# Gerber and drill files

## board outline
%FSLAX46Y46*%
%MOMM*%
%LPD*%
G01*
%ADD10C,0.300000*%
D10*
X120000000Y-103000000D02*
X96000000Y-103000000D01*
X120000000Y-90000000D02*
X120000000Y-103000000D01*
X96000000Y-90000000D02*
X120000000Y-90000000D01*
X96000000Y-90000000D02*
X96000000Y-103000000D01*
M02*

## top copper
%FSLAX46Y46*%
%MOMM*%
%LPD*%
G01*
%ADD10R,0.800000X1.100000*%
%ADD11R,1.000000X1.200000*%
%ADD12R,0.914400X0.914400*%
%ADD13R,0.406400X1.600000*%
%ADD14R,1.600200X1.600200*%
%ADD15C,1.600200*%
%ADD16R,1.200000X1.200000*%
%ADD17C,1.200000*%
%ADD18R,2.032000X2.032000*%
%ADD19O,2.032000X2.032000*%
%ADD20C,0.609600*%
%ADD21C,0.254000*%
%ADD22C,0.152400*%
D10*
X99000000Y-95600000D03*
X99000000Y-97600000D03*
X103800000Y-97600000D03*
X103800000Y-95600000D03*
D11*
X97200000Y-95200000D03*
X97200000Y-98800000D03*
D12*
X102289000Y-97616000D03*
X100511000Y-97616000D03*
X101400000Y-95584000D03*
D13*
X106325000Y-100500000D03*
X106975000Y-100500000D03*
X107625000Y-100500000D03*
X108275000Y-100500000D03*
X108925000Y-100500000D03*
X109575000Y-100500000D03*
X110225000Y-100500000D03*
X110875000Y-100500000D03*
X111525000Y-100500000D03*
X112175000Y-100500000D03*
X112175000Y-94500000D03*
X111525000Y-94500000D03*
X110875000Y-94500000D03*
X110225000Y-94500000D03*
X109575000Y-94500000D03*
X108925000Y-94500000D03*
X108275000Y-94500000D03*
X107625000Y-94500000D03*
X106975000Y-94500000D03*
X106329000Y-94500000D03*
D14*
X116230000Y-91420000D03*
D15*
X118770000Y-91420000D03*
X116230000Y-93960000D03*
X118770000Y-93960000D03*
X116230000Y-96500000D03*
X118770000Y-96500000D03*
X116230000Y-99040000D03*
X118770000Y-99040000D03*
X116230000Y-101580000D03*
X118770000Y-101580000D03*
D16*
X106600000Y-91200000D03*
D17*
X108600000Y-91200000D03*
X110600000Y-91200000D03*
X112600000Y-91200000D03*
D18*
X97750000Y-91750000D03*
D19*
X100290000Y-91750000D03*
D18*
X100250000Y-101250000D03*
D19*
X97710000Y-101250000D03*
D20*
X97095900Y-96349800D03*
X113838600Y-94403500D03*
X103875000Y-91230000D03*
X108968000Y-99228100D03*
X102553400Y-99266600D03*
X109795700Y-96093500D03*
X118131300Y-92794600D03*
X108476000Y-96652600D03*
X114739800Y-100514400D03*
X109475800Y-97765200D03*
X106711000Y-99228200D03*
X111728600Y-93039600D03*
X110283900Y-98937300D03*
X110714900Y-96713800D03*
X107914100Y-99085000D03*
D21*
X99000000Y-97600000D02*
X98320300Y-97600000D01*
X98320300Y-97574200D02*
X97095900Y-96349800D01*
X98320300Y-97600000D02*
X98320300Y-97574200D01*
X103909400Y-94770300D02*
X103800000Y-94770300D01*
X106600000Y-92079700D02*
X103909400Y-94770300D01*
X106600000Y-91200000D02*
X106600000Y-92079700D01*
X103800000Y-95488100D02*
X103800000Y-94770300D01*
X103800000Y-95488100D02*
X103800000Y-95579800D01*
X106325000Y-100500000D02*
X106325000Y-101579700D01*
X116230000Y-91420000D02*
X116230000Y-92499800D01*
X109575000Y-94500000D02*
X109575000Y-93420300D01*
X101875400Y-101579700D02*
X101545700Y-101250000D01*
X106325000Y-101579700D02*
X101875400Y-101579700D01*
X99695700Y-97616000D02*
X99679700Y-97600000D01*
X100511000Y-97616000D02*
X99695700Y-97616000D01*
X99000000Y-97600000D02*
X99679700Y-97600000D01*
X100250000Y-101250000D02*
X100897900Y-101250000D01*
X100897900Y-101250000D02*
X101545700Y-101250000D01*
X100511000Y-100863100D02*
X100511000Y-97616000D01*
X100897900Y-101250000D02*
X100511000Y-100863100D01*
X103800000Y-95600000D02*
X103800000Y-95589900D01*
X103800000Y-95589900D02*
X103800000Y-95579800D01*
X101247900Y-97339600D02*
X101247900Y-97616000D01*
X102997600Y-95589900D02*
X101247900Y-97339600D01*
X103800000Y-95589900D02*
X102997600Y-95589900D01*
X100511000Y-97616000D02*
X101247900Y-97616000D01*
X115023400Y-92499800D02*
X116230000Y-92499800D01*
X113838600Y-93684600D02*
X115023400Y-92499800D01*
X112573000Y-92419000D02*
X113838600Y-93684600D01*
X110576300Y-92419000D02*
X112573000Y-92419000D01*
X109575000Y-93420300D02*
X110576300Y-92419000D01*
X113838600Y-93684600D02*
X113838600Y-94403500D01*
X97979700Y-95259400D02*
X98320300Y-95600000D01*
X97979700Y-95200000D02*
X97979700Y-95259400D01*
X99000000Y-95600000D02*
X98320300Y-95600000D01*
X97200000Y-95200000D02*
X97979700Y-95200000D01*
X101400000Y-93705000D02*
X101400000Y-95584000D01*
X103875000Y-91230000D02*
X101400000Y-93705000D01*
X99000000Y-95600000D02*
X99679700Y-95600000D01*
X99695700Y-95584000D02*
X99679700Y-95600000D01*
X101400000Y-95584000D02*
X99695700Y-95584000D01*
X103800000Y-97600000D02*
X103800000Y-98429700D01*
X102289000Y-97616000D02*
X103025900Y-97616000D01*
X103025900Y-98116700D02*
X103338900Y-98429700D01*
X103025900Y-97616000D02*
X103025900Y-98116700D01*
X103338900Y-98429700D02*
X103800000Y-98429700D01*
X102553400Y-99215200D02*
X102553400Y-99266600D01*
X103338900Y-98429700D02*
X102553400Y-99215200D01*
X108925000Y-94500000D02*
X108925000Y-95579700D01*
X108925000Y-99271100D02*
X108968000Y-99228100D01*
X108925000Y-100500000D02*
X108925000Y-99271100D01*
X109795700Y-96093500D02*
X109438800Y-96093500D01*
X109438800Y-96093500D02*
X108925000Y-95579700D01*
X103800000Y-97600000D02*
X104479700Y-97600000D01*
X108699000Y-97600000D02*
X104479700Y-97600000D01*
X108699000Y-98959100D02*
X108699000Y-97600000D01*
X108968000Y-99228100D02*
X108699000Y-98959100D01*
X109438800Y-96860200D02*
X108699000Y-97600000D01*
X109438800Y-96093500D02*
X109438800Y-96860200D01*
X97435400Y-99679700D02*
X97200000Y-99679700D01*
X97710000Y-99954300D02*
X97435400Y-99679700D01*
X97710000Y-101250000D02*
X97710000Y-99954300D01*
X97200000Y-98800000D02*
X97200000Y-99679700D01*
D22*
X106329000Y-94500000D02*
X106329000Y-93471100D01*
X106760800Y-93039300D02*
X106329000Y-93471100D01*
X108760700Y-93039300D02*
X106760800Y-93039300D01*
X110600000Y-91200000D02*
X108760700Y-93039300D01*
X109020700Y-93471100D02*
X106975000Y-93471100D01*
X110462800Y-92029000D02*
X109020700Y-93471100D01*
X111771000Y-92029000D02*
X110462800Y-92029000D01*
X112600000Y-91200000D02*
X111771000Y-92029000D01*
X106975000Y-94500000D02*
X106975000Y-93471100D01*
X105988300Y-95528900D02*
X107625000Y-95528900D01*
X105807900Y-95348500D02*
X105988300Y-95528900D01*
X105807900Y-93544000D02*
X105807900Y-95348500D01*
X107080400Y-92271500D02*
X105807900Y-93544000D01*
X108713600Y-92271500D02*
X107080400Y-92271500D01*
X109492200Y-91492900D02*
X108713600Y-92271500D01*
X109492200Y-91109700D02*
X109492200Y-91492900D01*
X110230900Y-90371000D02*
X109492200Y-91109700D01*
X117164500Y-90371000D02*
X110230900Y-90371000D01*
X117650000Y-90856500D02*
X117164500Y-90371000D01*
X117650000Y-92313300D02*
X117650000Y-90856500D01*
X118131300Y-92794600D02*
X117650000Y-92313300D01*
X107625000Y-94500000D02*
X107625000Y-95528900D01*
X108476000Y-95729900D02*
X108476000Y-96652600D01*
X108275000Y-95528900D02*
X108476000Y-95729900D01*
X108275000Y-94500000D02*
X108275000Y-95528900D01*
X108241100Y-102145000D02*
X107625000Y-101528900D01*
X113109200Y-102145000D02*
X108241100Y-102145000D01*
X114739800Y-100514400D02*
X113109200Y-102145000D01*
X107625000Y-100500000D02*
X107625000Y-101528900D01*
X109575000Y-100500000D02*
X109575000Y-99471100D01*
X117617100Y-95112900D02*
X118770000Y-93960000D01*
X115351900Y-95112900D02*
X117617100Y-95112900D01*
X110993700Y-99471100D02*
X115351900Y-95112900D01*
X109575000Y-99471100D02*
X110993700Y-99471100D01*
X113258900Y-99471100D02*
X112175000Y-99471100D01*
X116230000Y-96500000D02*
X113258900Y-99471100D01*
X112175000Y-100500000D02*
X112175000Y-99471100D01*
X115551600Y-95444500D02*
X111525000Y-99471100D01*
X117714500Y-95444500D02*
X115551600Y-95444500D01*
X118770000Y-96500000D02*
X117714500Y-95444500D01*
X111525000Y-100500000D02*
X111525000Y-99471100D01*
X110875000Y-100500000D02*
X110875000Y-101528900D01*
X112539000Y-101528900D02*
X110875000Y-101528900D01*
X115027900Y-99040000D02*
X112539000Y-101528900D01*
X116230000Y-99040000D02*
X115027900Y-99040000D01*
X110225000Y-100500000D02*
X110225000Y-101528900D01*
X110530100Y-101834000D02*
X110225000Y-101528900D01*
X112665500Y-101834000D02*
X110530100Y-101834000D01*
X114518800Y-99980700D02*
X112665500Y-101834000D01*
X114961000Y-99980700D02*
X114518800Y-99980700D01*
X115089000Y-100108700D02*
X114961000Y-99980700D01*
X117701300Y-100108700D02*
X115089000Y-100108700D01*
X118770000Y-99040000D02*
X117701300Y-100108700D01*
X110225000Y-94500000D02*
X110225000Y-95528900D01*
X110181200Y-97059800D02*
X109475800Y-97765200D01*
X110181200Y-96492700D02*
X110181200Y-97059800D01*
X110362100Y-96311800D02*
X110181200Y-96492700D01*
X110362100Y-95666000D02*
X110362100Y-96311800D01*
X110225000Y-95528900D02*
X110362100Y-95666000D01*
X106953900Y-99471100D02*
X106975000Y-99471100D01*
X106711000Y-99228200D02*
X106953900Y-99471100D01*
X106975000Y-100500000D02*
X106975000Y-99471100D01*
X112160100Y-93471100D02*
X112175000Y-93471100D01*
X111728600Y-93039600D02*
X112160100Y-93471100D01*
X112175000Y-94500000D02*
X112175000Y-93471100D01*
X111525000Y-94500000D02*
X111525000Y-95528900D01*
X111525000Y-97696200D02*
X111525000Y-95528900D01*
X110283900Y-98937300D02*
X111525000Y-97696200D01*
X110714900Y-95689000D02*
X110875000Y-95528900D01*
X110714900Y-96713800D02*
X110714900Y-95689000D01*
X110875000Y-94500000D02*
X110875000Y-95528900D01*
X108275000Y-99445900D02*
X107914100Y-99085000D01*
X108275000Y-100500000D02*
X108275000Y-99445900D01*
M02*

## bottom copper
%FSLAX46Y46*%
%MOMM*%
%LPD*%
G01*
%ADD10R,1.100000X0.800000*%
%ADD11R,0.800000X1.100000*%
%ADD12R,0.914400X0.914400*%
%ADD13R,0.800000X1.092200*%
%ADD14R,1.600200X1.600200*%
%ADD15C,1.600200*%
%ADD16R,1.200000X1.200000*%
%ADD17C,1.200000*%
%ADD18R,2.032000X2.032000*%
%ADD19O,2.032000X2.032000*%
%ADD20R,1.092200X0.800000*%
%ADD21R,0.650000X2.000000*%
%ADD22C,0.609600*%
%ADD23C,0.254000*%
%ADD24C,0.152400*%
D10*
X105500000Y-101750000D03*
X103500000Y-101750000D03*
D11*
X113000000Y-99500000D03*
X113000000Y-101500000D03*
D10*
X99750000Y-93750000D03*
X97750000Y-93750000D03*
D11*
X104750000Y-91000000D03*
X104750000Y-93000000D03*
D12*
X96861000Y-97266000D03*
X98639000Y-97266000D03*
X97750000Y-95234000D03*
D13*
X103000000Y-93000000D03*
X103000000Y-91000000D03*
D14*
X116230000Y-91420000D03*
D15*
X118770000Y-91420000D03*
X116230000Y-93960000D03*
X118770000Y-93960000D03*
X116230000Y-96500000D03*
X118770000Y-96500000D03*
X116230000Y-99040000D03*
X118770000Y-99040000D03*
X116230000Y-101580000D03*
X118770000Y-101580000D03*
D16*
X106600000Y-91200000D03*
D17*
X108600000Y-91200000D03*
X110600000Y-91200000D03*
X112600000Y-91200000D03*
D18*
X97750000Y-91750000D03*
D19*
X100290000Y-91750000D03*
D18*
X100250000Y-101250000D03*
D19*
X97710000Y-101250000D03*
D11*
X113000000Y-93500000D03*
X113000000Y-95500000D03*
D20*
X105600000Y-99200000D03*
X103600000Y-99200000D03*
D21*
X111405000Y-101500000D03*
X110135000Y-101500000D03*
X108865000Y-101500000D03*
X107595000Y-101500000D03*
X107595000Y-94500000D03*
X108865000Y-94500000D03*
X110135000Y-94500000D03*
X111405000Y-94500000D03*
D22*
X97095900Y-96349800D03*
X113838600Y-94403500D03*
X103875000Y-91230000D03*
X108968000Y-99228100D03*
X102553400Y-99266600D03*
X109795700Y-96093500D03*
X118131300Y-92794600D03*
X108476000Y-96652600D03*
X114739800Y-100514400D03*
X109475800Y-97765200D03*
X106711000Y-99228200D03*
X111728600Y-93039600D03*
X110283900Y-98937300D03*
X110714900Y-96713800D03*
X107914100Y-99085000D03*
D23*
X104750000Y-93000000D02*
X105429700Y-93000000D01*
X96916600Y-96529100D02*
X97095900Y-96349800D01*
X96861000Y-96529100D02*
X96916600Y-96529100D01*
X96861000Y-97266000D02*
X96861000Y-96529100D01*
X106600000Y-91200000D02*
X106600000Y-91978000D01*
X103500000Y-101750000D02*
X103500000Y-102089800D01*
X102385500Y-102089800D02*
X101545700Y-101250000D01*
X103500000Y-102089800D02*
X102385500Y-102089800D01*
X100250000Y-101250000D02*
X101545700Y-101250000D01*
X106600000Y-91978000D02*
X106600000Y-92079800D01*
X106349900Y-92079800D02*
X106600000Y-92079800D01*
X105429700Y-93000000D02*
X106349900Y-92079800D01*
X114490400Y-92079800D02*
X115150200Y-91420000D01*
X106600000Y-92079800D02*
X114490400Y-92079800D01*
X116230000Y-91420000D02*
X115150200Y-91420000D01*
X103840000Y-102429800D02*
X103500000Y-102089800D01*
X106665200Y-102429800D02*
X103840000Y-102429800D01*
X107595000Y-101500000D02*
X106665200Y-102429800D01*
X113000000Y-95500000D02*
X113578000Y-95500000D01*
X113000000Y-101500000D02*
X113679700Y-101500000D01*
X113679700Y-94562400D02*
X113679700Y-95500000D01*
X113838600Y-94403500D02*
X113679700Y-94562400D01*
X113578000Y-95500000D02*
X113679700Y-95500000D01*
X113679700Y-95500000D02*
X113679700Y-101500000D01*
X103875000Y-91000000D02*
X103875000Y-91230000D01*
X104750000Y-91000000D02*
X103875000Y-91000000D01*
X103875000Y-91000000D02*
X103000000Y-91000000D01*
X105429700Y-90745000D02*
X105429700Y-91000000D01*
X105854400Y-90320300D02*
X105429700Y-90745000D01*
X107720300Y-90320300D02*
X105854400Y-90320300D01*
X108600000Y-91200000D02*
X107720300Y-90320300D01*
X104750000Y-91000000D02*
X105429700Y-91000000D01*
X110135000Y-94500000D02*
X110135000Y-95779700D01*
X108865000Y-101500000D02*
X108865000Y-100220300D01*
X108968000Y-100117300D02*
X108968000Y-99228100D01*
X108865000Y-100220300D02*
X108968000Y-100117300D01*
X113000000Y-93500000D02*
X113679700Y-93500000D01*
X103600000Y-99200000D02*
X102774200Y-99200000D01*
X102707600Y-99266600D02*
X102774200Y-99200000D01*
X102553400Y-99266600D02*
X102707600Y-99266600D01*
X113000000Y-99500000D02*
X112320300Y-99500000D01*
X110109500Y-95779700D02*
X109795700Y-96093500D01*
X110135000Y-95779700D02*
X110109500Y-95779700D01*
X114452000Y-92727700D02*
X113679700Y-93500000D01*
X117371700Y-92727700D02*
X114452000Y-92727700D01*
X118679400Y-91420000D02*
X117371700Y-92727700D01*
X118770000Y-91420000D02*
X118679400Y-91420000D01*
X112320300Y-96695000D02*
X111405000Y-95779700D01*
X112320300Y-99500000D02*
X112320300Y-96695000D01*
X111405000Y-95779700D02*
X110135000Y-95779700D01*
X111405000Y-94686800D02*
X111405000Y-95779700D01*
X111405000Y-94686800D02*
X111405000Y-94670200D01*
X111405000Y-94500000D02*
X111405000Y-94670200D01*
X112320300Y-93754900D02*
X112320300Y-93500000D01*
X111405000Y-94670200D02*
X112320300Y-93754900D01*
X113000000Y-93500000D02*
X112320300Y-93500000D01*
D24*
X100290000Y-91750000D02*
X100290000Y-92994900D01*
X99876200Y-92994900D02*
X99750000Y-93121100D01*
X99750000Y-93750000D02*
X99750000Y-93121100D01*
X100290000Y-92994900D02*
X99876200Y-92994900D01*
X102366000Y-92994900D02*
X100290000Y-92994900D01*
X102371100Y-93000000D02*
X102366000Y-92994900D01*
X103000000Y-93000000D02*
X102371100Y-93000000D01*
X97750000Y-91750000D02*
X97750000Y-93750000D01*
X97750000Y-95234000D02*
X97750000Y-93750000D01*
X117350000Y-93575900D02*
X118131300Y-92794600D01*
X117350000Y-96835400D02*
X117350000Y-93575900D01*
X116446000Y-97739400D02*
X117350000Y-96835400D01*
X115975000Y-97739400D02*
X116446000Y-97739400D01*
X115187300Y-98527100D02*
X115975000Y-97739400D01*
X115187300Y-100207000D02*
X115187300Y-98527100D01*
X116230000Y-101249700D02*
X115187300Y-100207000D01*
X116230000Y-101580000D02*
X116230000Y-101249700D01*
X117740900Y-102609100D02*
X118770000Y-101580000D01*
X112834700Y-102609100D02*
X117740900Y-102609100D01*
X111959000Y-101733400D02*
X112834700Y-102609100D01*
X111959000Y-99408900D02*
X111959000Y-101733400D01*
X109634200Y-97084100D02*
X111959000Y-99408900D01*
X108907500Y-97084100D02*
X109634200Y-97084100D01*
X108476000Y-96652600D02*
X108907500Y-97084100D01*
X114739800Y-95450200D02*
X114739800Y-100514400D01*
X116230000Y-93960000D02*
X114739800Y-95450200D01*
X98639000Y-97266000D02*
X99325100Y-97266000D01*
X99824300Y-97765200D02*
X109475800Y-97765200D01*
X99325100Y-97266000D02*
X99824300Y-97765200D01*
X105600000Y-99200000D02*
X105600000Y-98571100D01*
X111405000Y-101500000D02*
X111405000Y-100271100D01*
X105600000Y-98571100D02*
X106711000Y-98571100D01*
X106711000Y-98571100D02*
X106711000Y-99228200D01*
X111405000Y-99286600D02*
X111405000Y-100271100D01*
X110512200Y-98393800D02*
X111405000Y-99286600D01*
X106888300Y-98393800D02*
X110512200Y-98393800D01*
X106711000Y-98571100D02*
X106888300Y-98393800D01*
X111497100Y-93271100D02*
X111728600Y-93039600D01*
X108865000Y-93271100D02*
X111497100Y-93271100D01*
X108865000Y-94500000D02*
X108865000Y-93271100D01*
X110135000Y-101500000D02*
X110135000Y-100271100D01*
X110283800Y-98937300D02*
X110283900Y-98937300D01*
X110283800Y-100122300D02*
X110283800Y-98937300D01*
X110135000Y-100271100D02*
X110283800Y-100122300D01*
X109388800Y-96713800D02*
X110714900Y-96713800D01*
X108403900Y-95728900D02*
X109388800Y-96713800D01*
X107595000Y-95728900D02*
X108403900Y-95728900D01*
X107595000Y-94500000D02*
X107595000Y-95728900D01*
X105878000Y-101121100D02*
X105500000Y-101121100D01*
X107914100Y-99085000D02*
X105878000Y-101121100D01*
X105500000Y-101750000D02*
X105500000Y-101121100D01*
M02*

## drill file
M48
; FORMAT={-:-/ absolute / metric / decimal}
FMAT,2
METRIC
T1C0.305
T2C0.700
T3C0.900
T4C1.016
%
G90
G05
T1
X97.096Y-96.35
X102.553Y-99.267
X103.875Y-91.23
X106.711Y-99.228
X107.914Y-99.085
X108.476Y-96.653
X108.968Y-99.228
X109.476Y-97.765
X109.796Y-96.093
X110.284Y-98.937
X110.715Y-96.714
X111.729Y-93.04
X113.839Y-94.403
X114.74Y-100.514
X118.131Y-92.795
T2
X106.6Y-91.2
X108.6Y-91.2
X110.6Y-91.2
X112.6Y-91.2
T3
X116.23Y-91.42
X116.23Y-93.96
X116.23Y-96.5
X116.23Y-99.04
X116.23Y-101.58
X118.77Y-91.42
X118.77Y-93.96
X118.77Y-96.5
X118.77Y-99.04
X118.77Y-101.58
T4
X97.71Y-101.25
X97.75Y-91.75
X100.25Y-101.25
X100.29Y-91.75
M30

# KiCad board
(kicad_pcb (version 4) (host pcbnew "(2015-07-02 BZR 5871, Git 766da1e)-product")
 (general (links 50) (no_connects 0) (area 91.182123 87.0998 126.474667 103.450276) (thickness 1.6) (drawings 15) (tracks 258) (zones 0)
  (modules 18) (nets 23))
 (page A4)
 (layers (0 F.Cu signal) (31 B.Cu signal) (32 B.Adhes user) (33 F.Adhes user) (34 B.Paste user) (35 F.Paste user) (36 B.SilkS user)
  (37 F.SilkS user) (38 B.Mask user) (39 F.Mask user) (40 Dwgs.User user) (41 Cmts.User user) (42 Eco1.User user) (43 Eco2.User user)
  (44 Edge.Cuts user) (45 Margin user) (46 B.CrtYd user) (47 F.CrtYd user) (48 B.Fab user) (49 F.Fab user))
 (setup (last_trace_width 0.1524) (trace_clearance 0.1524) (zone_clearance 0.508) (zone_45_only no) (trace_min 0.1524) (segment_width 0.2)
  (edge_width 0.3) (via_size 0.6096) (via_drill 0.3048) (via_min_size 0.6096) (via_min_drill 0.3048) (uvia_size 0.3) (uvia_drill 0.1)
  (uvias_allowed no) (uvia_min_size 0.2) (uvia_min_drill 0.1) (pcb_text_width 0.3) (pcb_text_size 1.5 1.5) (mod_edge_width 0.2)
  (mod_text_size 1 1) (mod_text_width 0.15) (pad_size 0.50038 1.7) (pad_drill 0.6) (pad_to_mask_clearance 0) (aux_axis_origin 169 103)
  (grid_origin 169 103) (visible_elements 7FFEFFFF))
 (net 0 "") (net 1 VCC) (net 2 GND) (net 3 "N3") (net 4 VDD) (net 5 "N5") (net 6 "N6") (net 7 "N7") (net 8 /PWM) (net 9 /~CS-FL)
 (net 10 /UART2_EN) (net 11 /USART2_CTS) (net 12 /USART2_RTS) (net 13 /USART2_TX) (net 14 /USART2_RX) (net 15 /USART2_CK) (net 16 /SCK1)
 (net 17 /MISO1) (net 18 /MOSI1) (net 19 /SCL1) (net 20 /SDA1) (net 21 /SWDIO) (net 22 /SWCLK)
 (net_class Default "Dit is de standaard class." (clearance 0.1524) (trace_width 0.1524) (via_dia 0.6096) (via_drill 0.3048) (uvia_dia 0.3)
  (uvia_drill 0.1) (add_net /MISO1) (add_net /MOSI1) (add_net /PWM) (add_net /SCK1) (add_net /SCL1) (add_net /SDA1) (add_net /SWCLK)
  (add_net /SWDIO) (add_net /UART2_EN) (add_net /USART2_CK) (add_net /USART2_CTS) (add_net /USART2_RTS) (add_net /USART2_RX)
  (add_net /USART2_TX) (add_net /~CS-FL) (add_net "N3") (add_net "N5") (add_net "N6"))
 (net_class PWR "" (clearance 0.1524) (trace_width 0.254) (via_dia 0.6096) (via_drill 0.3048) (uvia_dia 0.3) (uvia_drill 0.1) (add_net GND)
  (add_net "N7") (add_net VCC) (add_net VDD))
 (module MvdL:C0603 (layer F.Cu) (at 99 96.6 270)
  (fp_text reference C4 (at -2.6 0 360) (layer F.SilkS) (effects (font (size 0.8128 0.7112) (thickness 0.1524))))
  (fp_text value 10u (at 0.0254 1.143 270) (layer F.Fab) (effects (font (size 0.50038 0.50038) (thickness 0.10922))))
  (pad 1 smd rect (at -1 0 270) (size 1.1 0.8) (layers F.Cu F.Paste F.Mask) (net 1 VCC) (clearance 0.1524))
  (pad 2 smd rect (at 1 0 270) (size 1.1 0.8) (layers F.Cu F.Paste F.Mask) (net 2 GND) (clearance 0.1524)))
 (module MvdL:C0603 (layer B.Cu) (at 104.5 101.75 180)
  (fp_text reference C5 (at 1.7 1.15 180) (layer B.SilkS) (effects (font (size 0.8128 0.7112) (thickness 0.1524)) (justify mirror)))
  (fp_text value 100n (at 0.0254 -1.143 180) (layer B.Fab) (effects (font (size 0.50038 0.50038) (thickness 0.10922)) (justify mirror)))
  (pad 1 smd rect (at -1 0 180) (size 1.1 0.8) (layers B.Cu B.Paste B.Mask) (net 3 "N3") (clearance 0.1524))
  (pad 2 smd rect (at 1 0 180) (size 1.1 0.8) (layers B.Cu B.Paste B.Mask) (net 2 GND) (clearance 0.1524)))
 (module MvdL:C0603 (layer F.Cu) (at 103.8 96.6 90)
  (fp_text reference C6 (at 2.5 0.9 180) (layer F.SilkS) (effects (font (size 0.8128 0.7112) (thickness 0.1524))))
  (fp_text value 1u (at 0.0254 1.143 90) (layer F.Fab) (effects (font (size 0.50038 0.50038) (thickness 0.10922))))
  (pad 1 smd rect (at -1 0 90) (size 1.1 0.8) (layers F.Cu F.Paste F.Mask) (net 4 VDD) (clearance 0.1524))
  (pad 2 smd rect (at 1 0 90) (size 1.1 0.8) (layers F.Cu F.Paste F.Mask) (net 2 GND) (clearance 0.1524)))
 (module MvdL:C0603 (layer B.Cu) (at 113 100.5 270)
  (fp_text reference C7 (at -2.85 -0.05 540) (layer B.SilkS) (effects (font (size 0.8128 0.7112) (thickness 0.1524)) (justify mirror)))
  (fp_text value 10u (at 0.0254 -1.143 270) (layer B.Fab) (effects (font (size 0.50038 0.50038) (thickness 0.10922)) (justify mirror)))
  (pad 1 smd rect (at -1 0 270) (size 1.1 0.8) (layers B.Cu B.Paste B.Mask) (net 4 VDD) (clearance 0.1524))
  (pad 2 smd rect (at 1 0 270) (size 1.1 0.8) (layers B.Cu B.Paste B.Mask) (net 2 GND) (clearance 0.1524)))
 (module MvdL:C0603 (layer B.Cu) (at 98.75 93.75 180)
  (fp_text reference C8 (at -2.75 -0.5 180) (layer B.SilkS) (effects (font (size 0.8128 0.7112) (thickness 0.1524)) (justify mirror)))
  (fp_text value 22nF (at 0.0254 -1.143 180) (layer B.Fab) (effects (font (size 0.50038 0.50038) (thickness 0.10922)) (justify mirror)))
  (pad 1 smd rect (at -1 0 180) (size 1.1 0.8) (layers B.Cu B.Paste B.Mask) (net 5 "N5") (clearance 0.1524))
  (pad 2 smd rect (at 1 0 180) (size 1.1 0.8) (layers B.Cu B.Paste B.Mask) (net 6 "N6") (clearance 0.1524)))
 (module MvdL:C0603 (layer B.Cu) (at 104.75 92 270)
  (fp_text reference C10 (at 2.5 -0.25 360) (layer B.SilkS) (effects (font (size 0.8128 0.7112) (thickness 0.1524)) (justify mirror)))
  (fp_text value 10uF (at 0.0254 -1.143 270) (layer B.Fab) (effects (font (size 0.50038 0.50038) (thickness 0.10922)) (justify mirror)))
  (pad 1 smd rect (at -1 0 270) (size 1.1 0.8) (layers B.Cu B.Paste B.Mask) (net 1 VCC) (clearance 0.1524))
  (pad 2 smd rect (at 1 0 270) (size 1.1 0.8) (layers B.Cu B.Paste B.Mask) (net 2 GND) (clearance 0.1524)))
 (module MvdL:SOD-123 (layer F.Cu) (at 97.2 97 270)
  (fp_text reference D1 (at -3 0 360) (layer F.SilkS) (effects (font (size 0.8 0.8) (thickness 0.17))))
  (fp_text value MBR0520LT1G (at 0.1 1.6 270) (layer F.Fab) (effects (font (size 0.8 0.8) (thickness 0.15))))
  (pad C smd rect (at -1.8 0 270) (size 1.2 1) (layers F.Cu F.Paste F.Mask) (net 1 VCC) (clearance 0.1524))
  (pad A smd rect (at 1.8 0 270) (size 1.2 1) (layers F.Cu F.Paste F.Mask) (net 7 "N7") (clearance 0.1524)))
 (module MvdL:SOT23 (layer B.Cu) (at 97.75 96.25)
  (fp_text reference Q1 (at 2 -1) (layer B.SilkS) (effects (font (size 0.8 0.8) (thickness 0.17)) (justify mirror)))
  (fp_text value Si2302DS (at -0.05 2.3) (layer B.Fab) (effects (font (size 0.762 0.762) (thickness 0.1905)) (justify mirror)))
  (pad 2 smd rect (at -0.889 1.016) (size 0.9144 0.9144) (layers B.Cu B.Paste B.Mask) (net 2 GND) (die_length -2147.483648)
   (clearance 0.1524))
  (pad 1 smd rect (at 0.889 1.016) (size 0.9144 0.9144) (layers B.Cu B.Paste B.Mask) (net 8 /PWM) (clearance 0.1524))
  (pad 3 smd rect (at 0 -1.016) (size 0.9144 0.9144) (layers B.Cu B.Paste B.Mask) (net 6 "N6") (clearance 0.1524)))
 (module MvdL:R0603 (layer B.Cu) (at 103 92 90)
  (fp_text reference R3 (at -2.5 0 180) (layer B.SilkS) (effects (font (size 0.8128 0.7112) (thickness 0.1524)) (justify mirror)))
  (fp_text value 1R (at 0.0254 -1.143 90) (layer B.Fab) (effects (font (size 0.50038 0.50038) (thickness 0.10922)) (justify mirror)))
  (pad 1 smd rect (at -1 0 90) (size 1.0922 0.8) (layers B.Cu B.Paste B.Mask) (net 5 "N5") (clearance 0.1524))
  (pad 2 smd rect (at 1 0 90) (size 1.0922 0.8) (layers B.Cu B.Paste B.Mask) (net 1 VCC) (clearance 0.1524)))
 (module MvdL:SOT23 (layer F.Cu) (at 101.4 96.6 180)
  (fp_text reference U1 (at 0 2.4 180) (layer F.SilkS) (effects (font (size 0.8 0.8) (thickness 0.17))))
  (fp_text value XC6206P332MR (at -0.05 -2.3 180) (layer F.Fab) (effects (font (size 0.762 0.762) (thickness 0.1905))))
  (pad 2 smd rect (at -0.889 -1.016 180) (size 0.9144 0.9144) (layers F.Cu F.Paste F.Mask) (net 4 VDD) (die_length -2147.483648)
   (clearance 0.1524))
  (pad 1 smd rect (at 0.889 -1.016 180) (size 0.9144 0.9144) (layers F.Cu F.Paste F.Mask) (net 2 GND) (clearance 0.1524))
  (pad 3 smd rect (at 0 1.016 180) (size 0.9144 0.9144) (layers F.Cu F.Paste F.Mask) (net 1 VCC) (clearance 0.1524)))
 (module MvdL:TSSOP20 (layer F.Cu) (at 109.25 97.5)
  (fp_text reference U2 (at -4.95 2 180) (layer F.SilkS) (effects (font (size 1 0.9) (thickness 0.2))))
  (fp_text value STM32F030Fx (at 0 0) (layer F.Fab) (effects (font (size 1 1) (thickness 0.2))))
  (pad 1 smd rect (at -2.925 3) (size 0.4064 1.6) (layers F.Cu F.Paste F.Mask) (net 2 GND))
  (pad 2 smd rect (at -2.275 3) (size 0.4064 1.6) (layers F.Cu F.Paste F.Mask) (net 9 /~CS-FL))
  (pad 3 smd rect (at -1.625 3) (size 0.4064 1.6) (layers F.Cu F.Paste F.Mask) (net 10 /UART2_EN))
  (pad 4 smd rect (at -0.975 3) (size 0.4064 1.6) (layers F.Cu F.Paste F.Mask) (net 3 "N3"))
  (pad 5 smd rect (at -0.325 3) (size 0.4064 1.6) (layers F.Cu F.Paste F.Mask) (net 4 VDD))
  (pad 6 smd rect (at 0.325 3) (size 0.4064 1.6) (layers F.Cu F.Paste F.Mask) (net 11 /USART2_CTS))
  (pad 7 smd rect (at 0.975 3) (size 0.4064 1.6) (layers F.Cu F.Paste F.Mask) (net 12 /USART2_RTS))
  (pad 8 smd rect (at 1.625 3) (size 0.4064 1.6) (layers F.Cu F.Paste F.Mask) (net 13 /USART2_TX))
  (pad 9 smd rect (at 2.275 3) (size 0.4064 1.6) (layers F.Cu F.Paste F.Mask) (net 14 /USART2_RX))
  (pad 10 smd rect (at 2.925 3) (size 0.4064 1.6) (layers F.Cu F.Paste F.Mask) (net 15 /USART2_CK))
  (pad 11 smd rect (at 2.925 -3) (size 0.4064 1.6) (layers F.Cu F.Paste F.Mask) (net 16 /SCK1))
  (pad 12 smd rect (at 2.275 -3) (size 0.4064 1.6) (layers F.Cu F.Paste F.Mask) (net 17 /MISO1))
  (pad 13 smd rect (at 1.625 -3) (size 0.4064 1.6) (layers F.Cu F.Paste F.Mask) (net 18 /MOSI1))
  (pad 14 smd rect (at 0.975 -3) (size 0.4064 1.6) (layers F.Cu F.Paste F.Mask) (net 8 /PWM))
  (pad 15 smd rect (at 0.325 -3) (size 0.4064 1.6) (layers F.Cu F.Paste F.Mask) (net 2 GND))
  (pad 16 smd rect (at -0.325 -3) (size 0.4064 1.6) (layers F.Cu F.Paste F.Mask) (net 4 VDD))
  (pad 17 smd rect (at -0.975 -3) (size 0.4064 1.6) (layers F.Cu F.Paste F.Mask) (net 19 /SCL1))
  (pad 18 smd rect (at -1.625 -3) (size 0.4064 1.6) (layers F.Cu F.Paste F.Mask) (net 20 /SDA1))
  (pad 19 smd rect (at -2.275 -3) (size 0.4064 1.6) (layers F.Cu F.Paste F.Mask) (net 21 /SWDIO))
  (pad 20 smd rect (at -2.921 -3) (size 0.4064 1.6) (layers F.Cu F.Paste F.Mask) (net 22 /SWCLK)))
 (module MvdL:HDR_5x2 (layer F.Cu) (at 117.5 96.5 270)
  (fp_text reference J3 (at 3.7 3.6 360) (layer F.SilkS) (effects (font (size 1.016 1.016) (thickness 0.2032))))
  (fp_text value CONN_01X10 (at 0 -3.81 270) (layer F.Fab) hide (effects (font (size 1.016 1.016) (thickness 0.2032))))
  (pad 1 thru_hole rect (at -5.08 1.27 270) (size 1.6002 1.6002) (drill 0.9) (layers *.Cu *.Mask F.SilkS) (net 2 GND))
  (pad 2 thru_hole circle (at -5.08 -1.27 270) (size 1.6002 1.6002) (drill 0.9) (layers *.Cu *.Mask F.SilkS) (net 4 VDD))
  (pad 3 thru_hole circle (at -2.54 1.27 270) (size 1.6002 1.6002) (drill 0.9) (layers *.Cu *.Mask F.SilkS) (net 10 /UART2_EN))
  (pad 4 thru_hole circle (at -2.54 -1.27 270) (size 1.6002 1.6002) (drill 0.9) (layers *.Cu *.Mask F.SilkS) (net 11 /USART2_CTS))
  (pad 5 thru_hole circle (at 0 1.27 270) (size 1.6002 1.6002) (drill 0.9) (layers *.Cu *.Mask F.SilkS) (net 15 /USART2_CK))
  (pad 6 thru_hole circle (at 0 -1.27 270) (size 1.6002 1.6002) (drill 0.9) (layers *.Cu *.Mask F.SilkS) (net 14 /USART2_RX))
  (pad 7 thru_hole circle (at 2.54 1.27 270) (size 1.6002 1.6002) (drill 0.9) (layers *.Cu *.Mask F.SilkS) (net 13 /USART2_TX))
  (pad 8 thru_hole circle (at 2.54 -1.27 270) (size 1.6002 1.6002) (drill 0.9) (layers *.Cu *.Mask F.SilkS) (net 12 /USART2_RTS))
  (pad 9 thru_hole circle (at 5.08 1.27 270) (size 1.6002 1.6002) (drill 0.9) (layers *.Cu *.Mask F.SilkS) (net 20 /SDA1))
  (pad 10 thru_hole circle (at 5.08 -1.27 270) (size 1.6002 1.6002) (drill 0.9) (layers *.Cu *.Mask F.SilkS) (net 19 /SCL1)))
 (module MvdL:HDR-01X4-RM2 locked (layer F.Cu) (at 106.6 91.2)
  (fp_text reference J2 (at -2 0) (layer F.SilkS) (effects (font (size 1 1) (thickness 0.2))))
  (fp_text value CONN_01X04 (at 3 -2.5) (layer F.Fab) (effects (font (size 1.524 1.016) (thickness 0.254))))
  (pad 1 thru_hole rect (at 0 0) (size 1.2 1.2) (drill 0.7) (layers *.Cu *.Mask F.SilkS) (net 2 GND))
  (pad 2 thru_hole circle (at 2 0) (size 1.2 1.2) (drill 0.7) (layers *.Cu *.Mask F.SilkS) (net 1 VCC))
  (pad 3 thru_hole circle (at 4 0) (size 1.2 1.2) (drill 0.7) (layers *.Cu *.Mask F.SilkS) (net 22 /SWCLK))
  (pad 4 thru_hole circle (at 6 0) (size 1.2 1.2) (drill 0.7) (layers *.Cu *.Mask F.SilkS) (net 21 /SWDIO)))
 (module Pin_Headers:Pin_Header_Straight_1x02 (layer F.Cu) (at 97.75 91.75 90)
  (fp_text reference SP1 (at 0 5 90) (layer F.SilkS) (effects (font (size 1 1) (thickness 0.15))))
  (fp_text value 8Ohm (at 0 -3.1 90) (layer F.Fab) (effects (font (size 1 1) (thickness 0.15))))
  (pad 1 thru_hole rect (at 0 0 90) (size 2.032 2.032) (drill 1.016) (layers *.Cu *.Mask F.SilkS) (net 6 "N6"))
  (pad 2 thru_hole oval (at 0 2.54 90) (size 2.032 2.032) (drill 1.016) (layers *.Cu *.Mask F.SilkS) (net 5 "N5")))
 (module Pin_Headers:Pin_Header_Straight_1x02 (layer F.Cu) (at 100.25 101.25 270)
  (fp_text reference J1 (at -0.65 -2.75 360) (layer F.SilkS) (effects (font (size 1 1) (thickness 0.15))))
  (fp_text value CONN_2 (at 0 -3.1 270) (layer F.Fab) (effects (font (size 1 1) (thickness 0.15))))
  (pad 1 thru_hole rect (at 0 0 270) (size 2.032 2.032) (drill 1.016) (layers *.Cu *.Mask F.SilkS) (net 2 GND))
  (pad 2 thru_hole oval (at 0 2.54 270) (size 2.032 2.032) (drill 1.016) (layers *.Cu *.Mask F.SilkS) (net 7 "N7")))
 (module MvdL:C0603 (layer B.Cu) (at 113 94.5 270)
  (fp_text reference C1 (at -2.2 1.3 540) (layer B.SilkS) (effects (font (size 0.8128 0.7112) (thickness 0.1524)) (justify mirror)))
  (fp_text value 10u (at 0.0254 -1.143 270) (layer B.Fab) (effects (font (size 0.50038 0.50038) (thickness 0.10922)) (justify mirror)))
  (pad 1 smd rect (at -1 0 270) (size 1.1 0.8) (layers B.Cu B.Paste B.Mask) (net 4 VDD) (clearance 0.1524))
  (pad 2 smd rect (at 1 0 270) (size 1.1 0.8) (layers B.Cu B.Paste B.Mask) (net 2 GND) (clearance 0.1524)))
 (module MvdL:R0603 (layer B.Cu) (at 104.6 99.2 180)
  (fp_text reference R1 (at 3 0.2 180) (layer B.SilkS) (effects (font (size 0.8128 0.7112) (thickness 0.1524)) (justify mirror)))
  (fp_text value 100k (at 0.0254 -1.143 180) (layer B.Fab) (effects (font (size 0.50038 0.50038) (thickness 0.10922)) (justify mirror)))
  (pad 1 smd rect (at -1 0 180) (size 1.0922 0.8) (layers B.Cu B.Paste B.Mask) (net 9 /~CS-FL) (clearance 0.1524))
  (pad 2 smd rect (at 1 0 180) (size 1.0922 0.8) (layers B.Cu B.Paste B.Mask) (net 4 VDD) (clearance 0.1524)))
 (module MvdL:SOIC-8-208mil (layer B.Cu) (at 109.5 98 90)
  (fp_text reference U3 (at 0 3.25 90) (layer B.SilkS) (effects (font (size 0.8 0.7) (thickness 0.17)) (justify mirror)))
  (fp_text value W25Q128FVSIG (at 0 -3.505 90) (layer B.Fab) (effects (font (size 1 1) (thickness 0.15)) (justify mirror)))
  (pad 1 smd rect (at -3.5 1.905 90) (size 2 0.65) (layers B.Cu B.Paste B.Mask) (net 9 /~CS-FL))
  (pad 2 smd rect (at -3.5 0.635 90) (size 2 0.65) (layers B.Cu B.Paste B.Mask) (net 17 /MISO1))
  (pad 3 smd rect (at -3.5 -0.635 90) (size 2 0.65) (layers B.Cu B.Paste B.Mask) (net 4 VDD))
  (pad 4 smd rect (at -3.5 -1.905 90) (size 2 0.65) (layers B.Cu B.Paste B.Mask) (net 2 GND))
  (pad 5 smd rect (at 3.5 -1.905 90) (size 2 0.65) (layers B.Cu B.Paste B.Mask) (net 18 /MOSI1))
  (pad 6 smd rect (at 3.5 -0.635 90) (size 2 0.65) (layers B.Cu B.Paste B.Mask) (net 16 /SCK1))
  (pad 7 smd rect (at 3.5 0.635 90) (size 2 0.65) (layers B.Cu B.Paste B.Mask) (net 4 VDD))
  (pad 8 smd rect (at 3.5 1.905 90) (size 2 0.65) (layers B.Cu B.Paste B.Mask) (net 4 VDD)))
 (gr_line (start 120 103) (end 96 103) (angle 90) (layer Edge.Cuts) (width 0.3))
 (gr_line (start 120 90) (end 120 103) (angle 90) (layer Edge.Cuts) (width 0.3))
 (gr_line (start 96 90) (end 120 90) (angle 90) (layer Edge.Cuts) (width 0.3))
 (gr_line (start 96 90) (end 96 103) (angle 90) (layer Edge.Cuts) (width 0.3))
 (via (at 97.0959 96.3498) (size 0.6096) (layers F.Cu B.Cu) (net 2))
 (via (at 113.8386 94.4035) (size 0.6096) (layers F.Cu B.Cu) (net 2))
 (segment (start 104.75 93) (end 105.4297 93) (width 0.254) (layer B.Cu) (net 2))
 (segment (start 99 97.6) (end 98.3203 97.6) (width 0.254) (layer F.Cu) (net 2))
 (segment (start 96.9166 96.5291) (end 97.0959 96.3498) (width 0.254) (layer B.Cu) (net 2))
 (segment (start 96.861 96.5291) (end 96.9166 96.5291) (width 0.254) (layer B.Cu) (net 2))
 (segment (start 98.3203 97.5742) (end 97.0959 96.3498) (width 0.254) (layer F.Cu) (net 2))
 (segment (start 98.3203 97.6) (end 98.3203 97.5742) (width 0.254) (layer F.Cu) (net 2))
 (segment (start 96.861 97.266) (end 96.861 96.5291) (width 0.254) (layer B.Cu) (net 2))
 (segment (start 103.9094 94.7703) (end 103.8 94.7703) (width 0.254) (layer F.Cu) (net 2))
 (segment (start 106.6 92.0797) (end 103.9094 94.7703) (width 0.254) (layer F.Cu) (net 2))
 (segment (start 106.6 91.2) (end 106.6 92.0797) (width 0.254) (layer F.Cu) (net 2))
 (segment (start 103.8 95.4881) (end 103.8 94.7703) (width 0.254) (layer F.Cu) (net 2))
 (segment (start 103.8 95.4881) (end 103.8 95.5798) (width 0.254) (layer F.Cu) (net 2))
 (segment (start 106.325 100.5) (end 106.325 101.5797) (width 0.254) (layer F.Cu) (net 2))
 (segment (start 106.6 91.2) (end 106.6 91.978) (width 0.254) (layer B.Cu) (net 2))
 (segment (start 116.23 91.42) (end 116.23 92.4998) (width 0.254) (layer F.Cu) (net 2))
 (segment (start 103.5 101.75) (end 103.5 102.0898) (width 0.254) (layer B.Cu) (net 2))
 (segment (start 102.3855 102.0898) (end 101.5457 101.25) (width 0.254) (layer B.Cu) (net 2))
 (segment (start 103.5 102.0898) (end 102.3855 102.0898) (width 0.254) (layer B.Cu) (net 2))
 (segment (start 100.25 101.25) (end 101.5457 101.25) (width 0.254) (layer B.Cu) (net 2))
 (segment (start 109.575 94.5) (end 109.575 93.4203) (width 0.254) (layer F.Cu) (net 2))
 (segment (start 106.6 91.978) (end 106.6 92.0798) (width 0.254) (layer B.Cu) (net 2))
 (segment (start 106.3499 92.0798) (end 106.6 92.0798) (width 0.254) (layer B.Cu) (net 2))
 (segment (start 105.4297 93) (end 106.3499 92.0798) (width 0.254) (layer B.Cu) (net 2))
 (segment (start 114.4904 92.0798) (end 115.1502 91.42) (width 0.254) (layer B.Cu) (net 2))
 (segment (start 106.6 92.0798) (end 114.4904 92.0798) (width 0.254) (layer B.Cu) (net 2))
 (segment (start 116.23 91.42) (end 115.1502 91.42) (width 0.254) (layer B.Cu) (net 2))
 (segment (start 103.84 102.4298) (end 103.5 102.0898) (width 0.254) (layer B.Cu) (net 2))
 (segment (start 106.6652 102.4298) (end 103.84 102.4298) (width 0.254) (layer B.Cu) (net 2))
 (segment (start 107.595 101.5) (end 106.6652 102.4298) (width 0.254) (layer B.Cu) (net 2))
 (segment (start 113 95.5) (end 113.578 95.5) (width 0.254) (layer B.Cu) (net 2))
 (segment (start 113 101.5) (end 113.6797 101.5) (width 0.254) (layer B.Cu) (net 2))
 (segment (start 101.8754 101.5797) (end 101.5457 101.25) (width 0.254) (layer F.Cu) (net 2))
 (segment (start 106.325 101.5797) (end 101.8754 101.5797) (width 0.254) (layer F.Cu) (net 2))
 (segment (start 99.6957 97.616) (end 99.6797 97.6) (width 0.254) (layer F.Cu) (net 2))
 (segment (start 100.511 97.616) (end 99.6957 97.616) (width 0.254) (layer F.Cu) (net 2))
 (segment (start 99 97.6) (end 99.6797 97.6) (width 0.254) (layer F.Cu) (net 2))
 (segment (start 100.25 101.25) (end 100.8979 101.25) (width 0.254) (layer F.Cu) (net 2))
 (segment (start 100.8979 101.25) (end 101.5457 101.25) (width 0.254) (layer F.Cu) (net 2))
 (segment (start 100.511 100.8631) (end 100.511 97.616) (width 0.254) (layer F.Cu) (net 2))
 (segment (start 100.8979 101.25) (end 100.511 100.8631) (width 0.254) (layer F.Cu) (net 2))
 (segment (start 103.8 95.6) (end 103.8 95.5899) (width 0.254) (layer F.Cu) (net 2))
 (segment (start 103.8 95.5899) (end 103.8 95.5798) (width 0.254) (layer F.Cu) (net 2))
 (segment (start 101.2479 97.3396) (end 101.2479 97.616) (width 0.254) (layer F.Cu) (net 2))
 (segment (start 102.9976 95.5899) (end 101.2479 97.3396) (width 0.254) (layer F.Cu) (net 2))
 (segment (start 103.8 95.5899) (end 102.9976 95.5899) (width 0.254) (layer F.Cu) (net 2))
 (segment (start 100.511 97.616) (end 101.2479 97.616) (width 0.254) (layer F.Cu) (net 2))
 (segment (start 113.6797 94.5624) (end 113.6797 95.5) (width 0.254) (layer B.Cu) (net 2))
 (segment (start 113.8386 94.4035) (end 113.6797 94.5624) (width 0.254) (layer B.Cu) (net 2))
 (segment (start 113.578 95.5) (end 113.6797 95.5) (width 0.254) (layer B.Cu) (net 2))
 (segment (start 113.6797 95.5) (end 113.6797 101.5) (width 0.254) (layer B.Cu) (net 2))
 (segment (start 115.0234 92.4998) (end 116.23 92.4998) (width 0.254) (layer F.Cu) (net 2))
 (segment (start 113.8386 93.6846) (end 115.0234 92.4998) (width 0.254) (layer F.Cu) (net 2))
 (segment (start 112.573 92.419) (end 113.8386 93.6846) (width 0.254) (layer F.Cu) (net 2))
 (segment (start 110.5763 92.419) (end 112.573 92.419) (width 0.254) (layer F.Cu) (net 2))
 (segment (start 109.575 93.4203) (end 110.5763 92.419) (width 0.254) (layer F.Cu) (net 2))
 (segment (start 113.8386 93.6846) (end 113.8386 94.4035) (width 0.254) (layer F.Cu) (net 2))
 (via (at 103.875 91.23) (size 0.6096) (layers F.Cu B.Cu) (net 1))
 (segment (start 97.9797 95.2594) (end 98.3203 95.6) (width 0.254) (layer F.Cu) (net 1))
 (segment (start 97.9797 95.2) (end 97.9797 95.2594) (width 0.254) (layer F.Cu) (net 1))
 (segment (start 99 95.6) (end 98.3203 95.6) (width 0.254) (layer F.Cu) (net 1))
 (segment (start 97.2 95.2) (end 97.9797 95.2) (width 0.254) (layer F.Cu) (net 1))
 (segment (start 103.875 91) (end 103.875 91.23) (width 0.254) (layer B.Cu) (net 1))
 (segment (start 104.75 91) (end 103.875 91) (width 0.254) (layer B.Cu) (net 1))
 (segment (start 103.875 91) (end 103 91) (width 0.254) (layer B.Cu) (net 1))
 (segment (start 101.4 93.705) (end 101.4 95.584) (width 0.254) (layer F.Cu) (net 1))
 (segment (start 103.875 91.23) (end 101.4 93.705) (width 0.254) (layer F.Cu) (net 1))
 (segment (start 99 95.6) (end 99.6797 95.6) (width 0.254) (layer F.Cu) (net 1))
 (segment (start 99.6957 95.584) (end 99.6797 95.6) (width 0.254) (layer F.Cu) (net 1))
 (segment (start 101.4 95.584) (end 99.6957 95.584) (width 0.254) (layer F.Cu) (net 1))
 (segment (start 105.4297 90.745) (end 105.4297 91) (width 0.254) (layer B.Cu) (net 1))
 (segment (start 105.8544 90.3203) (end 105.4297 90.745) (width 0.254) (layer B.Cu) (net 1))
 (segment (start 107.7203 90.3203) (end 105.8544 90.3203) (width 0.254) (layer B.Cu) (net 1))
 (segment (start 108.6 91.2) (end 107.7203 90.3203) (width 0.254) (layer B.Cu) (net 1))
 (segment (start 104.75 91) (end 105.4297 91) (width 0.254) (layer B.Cu) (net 1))
 (via (at 108.968 99.2281) (size 0.6096) (layers F.Cu B.Cu) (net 4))
 (via (at 102.5534 99.2666) (size 0.6096) (layers F.Cu B.Cu) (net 4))
 (via (at 109.7957 96.0935) (size 0.6096) (layers F.Cu B.Cu) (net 4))
 (segment (start 110.135 94.5) (end 110.135 95.7797) (width 0.254) (layer B.Cu) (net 4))
 (segment (start 108.865 101.5) (end 108.865 100.2203) (width 0.254) (layer B.Cu) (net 4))
 (segment (start 108.968 100.1173) (end 108.968 99.2281) (width 0.254) (layer B.Cu) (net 4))
 (segment (start 108.865 100.2203) (end 108.968 100.1173) (width 0.254) (layer B.Cu) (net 4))
 (segment (start 113 93.5) (end 113.6797 93.5) (width 0.254) (layer B.Cu) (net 4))
 (segment (start 103.8 97.6) (end 103.8 98.4297) (width 0.254) (layer F.Cu) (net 4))
 (segment (start 102.289 97.616) (end 103.0259 97.616) (width 0.254) (layer F.Cu) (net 4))
 (segment (start 103.0259 98.1167) (end 103.3389 98.4297) (width 0.254) (layer F.Cu) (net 4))
 (segment (start 103.0259 97.616) (end 103.0259 98.1167) (width 0.254) (layer F.Cu) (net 4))
 (segment (start 103.3389 98.4297) (end 103.8 98.4297) (width 0.254) (layer F.Cu) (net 4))
 (segment (start 103.6 99.2) (end 102.7742 99.2) (width 0.254) (layer B.Cu) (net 4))
 (segment (start 102.7076 99.2666) (end 102.7742 99.2) (width 0.254) (layer B.Cu) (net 4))
 (segment (start 102.5534 99.2666) (end 102.7076 99.2666) (width 0.254) (layer B.Cu) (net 4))
 (segment (start 102.5534 99.2152) (end 102.5534 99.2666) (width 0.254) (layer F.Cu) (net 4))
 (segment (start 103.3389 98.4297) (end 102.5534 99.2152) (width 0.254) (layer F.Cu) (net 4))
 (segment (start 113 99.5) (end 112.3203 99.5) (width 0.254) (layer B.Cu) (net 4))
 (segment (start 110.1095 95.7797) (end 109.7957 96.0935) (width 0.254) (layer B.Cu) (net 4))
 (segment (start 110.135 95.7797) (end 110.1095 95.7797) (width 0.254) (layer B.Cu) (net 4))
 (segment (start 108.925 94.5) (end 108.925 95.5797) (width 0.254) (layer F.Cu) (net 4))
 (segment (start 108.925 99.2711) (end 108.968 99.2281) (width 0.254) (layer F.Cu) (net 4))
 (segment (start 108.925 100.5) (end 108.925 99.2711) (width 0.254) (layer F.Cu) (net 4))
 (segment (start 109.7957 96.0935) (end 109.4388 96.0935) (width 0.254) (layer F.Cu) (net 4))
 (segment (start 109.4388 96.0935) (end 108.925 95.5797) (width 0.254) (layer F.Cu) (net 4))
 (segment (start 103.8 97.6) (end 104.4797 97.6) (width 0.254) (layer F.Cu) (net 4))
 (segment (start 108.699 97.6) (end 104.4797 97.6) (width 0.254) (layer F.Cu) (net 4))
 (segment (start 108.699 98.9591) (end 108.699 97.6) (width 0.254) (layer F.Cu) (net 4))
 (segment (start 108.968 99.2281) (end 108.699 98.9591) (width 0.254) (layer F.Cu) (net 4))
 (segment (start 114.452 92.7277) (end 113.6797 93.5) (width 0.254) (layer B.Cu) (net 4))
 (segment (start 117.3717 92.7277) (end 114.452 92.7277) (width 0.254) (layer B.Cu) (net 4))
 (segment (start 118.6794 91.42) (end 117.3717 92.7277) (width 0.254) (layer B.Cu) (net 4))
 (segment (start 118.77 91.42) (end 118.6794 91.42) (width 0.254) (layer B.Cu) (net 4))
 (segment (start 109.4388 96.8602) (end 108.699 97.6) (width 0.254) (layer F.Cu) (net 4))
 (segment (start 109.4388 96.0935) (end 109.4388 96.8602) (width 0.254) (layer F.Cu) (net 4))
 (segment (start 112.3203 96.695) (end 111.405 95.7797) (width 0.254) (layer B.Cu) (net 4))
 (segment (start 112.3203 99.5) (end 112.3203 96.695) (width 0.254) (layer B.Cu) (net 4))
 (segment (start 111.405 95.7797) (end 110.135 95.7797) (width 0.254) (layer B.Cu) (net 4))
 (segment (start 111.405 94.6868) (end 111.405 95.7797) (width 0.254) (layer B.Cu) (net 4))
 (segment (start 111.405 94.6868) (end 111.405 94.6702) (width 0.254) (layer B.Cu) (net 4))
 (segment (start 111.405 94.5) (end 111.405 94.6702) (width 0.254) (layer B.Cu) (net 4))
 (segment (start 112.3203 93.7549) (end 112.3203 93.5) (width 0.254) (layer B.Cu) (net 4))
 (segment (start 111.405 94.6702) (end 112.3203 93.7549) (width 0.254) (layer B.Cu) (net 4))
 (segment (start 113 93.5) (end 112.3203 93.5) (width 0.254) (layer B.Cu) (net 4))
 (segment (start 100.29 91.75) (end 100.29 92.9949) (width 0.1524) (layer B.Cu) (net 5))
 (segment (start 99.8762 92.9949) (end 99.75 93.1211) (width 0.1524) (layer B.Cu) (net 5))
 (segment (start 99.75 93.75) (end 99.75 93.1211) (width 0.1524) (layer B.Cu) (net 5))
 (segment (start 100.29 92.9949) (end 99.8762 92.9949) (width 0.1524) (layer B.Cu) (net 5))
 (segment (start 102.366 92.9949) (end 100.29 92.9949) (width 0.1524) (layer B.Cu) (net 5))
 (segment (start 102.3711 93) (end 102.366 92.9949) (width 0.1524) (layer B.Cu) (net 5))
 (segment (start 103 93) (end 102.3711 93) (width 0.1524) (layer B.Cu) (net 5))
 (segment (start 97.75 91.75) (end 97.75 93.75) (width 0.1524) (layer B.Cu) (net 6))
 (segment (start 97.75 95.234) (end 97.75 93.75) (width 0.1524) (layer B.Cu) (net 6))
 (segment (start 97.4354 99.6797) (end 97.2 99.6797) (width 0.254) (layer F.Cu) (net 7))
 (segment (start 97.71 99.9543) (end 97.4354 99.6797) (width 0.254) (layer F.Cu) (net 7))
 (segment (start 97.71 101.25) (end 97.71 99.9543) (width 0.254) (layer F.Cu) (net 7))
 (segment (start 97.2 98.8) (end 97.2 99.6797) (width 0.254) (layer F.Cu) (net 7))
 (segment (start 106.329 94.5) (end 106.329 93.4711) (width 0.1524) (layer F.Cu) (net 22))
 (segment (start 106.7608 93.0393) (end 106.329 93.4711) (width 0.1524) (layer F.Cu) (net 22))
 (segment (start 108.7607 93.0393) (end 106.7608 93.0393) (width 0.1524) (layer F.Cu) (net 22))
 (segment (start 110.6 91.2) (end 108.7607 93.0393) (width 0.1524) (layer F.Cu) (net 22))
 (segment (start 109.0207 93.4711) (end 106.975 93.4711) (width 0.1524) (layer F.Cu) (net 21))
 (segment (start 110.4628 92.029) (end 109.0207 93.4711) (width 0.1524) (layer F.Cu) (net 21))
 (segment (start 111.771 92.029) (end 110.4628 92.029) (width 0.1524) (layer F.Cu) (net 21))
 (segment (start 112.6 91.2) (end 111.771 92.029) (width 0.1524) (layer F.Cu) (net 21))
 (segment (start 106.975 94.5) (end 106.975 93.4711) (width 0.1524) (layer F.Cu) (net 21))
 (via (at 118.1313 92.7946) (size 0.6096) (layers F.Cu B.Cu) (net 20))
 (segment (start 105.9883 95.5289) (end 107.625 95.5289) (width 0.1524) (layer F.Cu) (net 20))
 (segment (start 105.8079 95.3485) (end 105.9883 95.5289) (width 0.1524) (layer F.Cu) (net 20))
 (segment (start 105.8079 93.544) (end 105.8079 95.3485) (width 0.1524) (layer F.Cu) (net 20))
 (segment (start 107.0804 92.2715) (end 105.8079 93.544) (width 0.1524) (layer F.Cu) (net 20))
 (segment (start 108.7136 92.2715) (end 107.0804 92.2715) (width 0.1524) (layer F.Cu) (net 20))
 (segment (start 109.4922 91.4929) (end 108.7136 92.2715) (width 0.1524) (layer F.Cu) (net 20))
 (segment (start 109.4922 91.1097) (end 109.4922 91.4929) (width 0.1524) (layer F.Cu) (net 20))
 (segment (start 110.2309 90.371) (end 109.4922 91.1097) (width 0.1524) (layer F.Cu) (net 20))
 (segment (start 117.1645 90.371) (end 110.2309 90.371) (width 0.1524) (layer F.Cu) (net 20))
 (segment (start 117.65 90.8565) (end 117.1645 90.371) (width 0.1524) (layer F.Cu) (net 20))
 (segment (start 117.65 92.3133) (end 117.65 90.8565) (width 0.1524) (layer F.Cu) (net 20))
 (segment (start 118.1313 92.7946) (end 117.65 92.3133) (width 0.1524) (layer F.Cu) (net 20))
 (segment (start 107.625 94.5) (end 107.625 95.5289) (width 0.1524) (layer F.Cu) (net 20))
 (segment (start 117.35 93.5759) (end 118.1313 92.7946) (width 0.1524) (layer B.Cu) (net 20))
 (segment (start 117.35 96.8354) (end 117.35 93.5759) (width 0.1524) (layer B.Cu) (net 20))
 (segment (start 116.446 97.7394) (end 117.35 96.8354) (width 0.1524) (layer B.Cu) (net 20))
 (segment (start 115.975 97.7394) (end 116.446 97.7394) (width 0.1524) (layer B.Cu) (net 20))
 (segment (start 115.1873 98.5271) (end 115.975 97.7394) (width 0.1524) (layer B.Cu) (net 20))
 (segment (start 115.1873 100.207) (end 115.1873 98.5271) (width 0.1524) (layer B.Cu) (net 20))
 (segment (start 116.23 101.2497) (end 115.1873 100.207) (width 0.1524) (layer B.Cu) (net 20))
 (segment (start 116.23 101.58) (end 116.23 101.2497) (width 0.1524) (layer B.Cu) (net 20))
 (via (at 108.476 96.6526) (size 0.6096) (layers F.Cu B.Cu) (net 19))
 (segment (start 108.476 95.7299) (end 108.476 96.6526) (width 0.1524) (layer F.Cu) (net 19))
 (segment (start 108.275 95.5289) (end 108.476 95.7299) (width 0.1524) (layer F.Cu) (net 19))
 (segment (start 117.7409 102.6091) (end 118.77 101.58) (width 0.1524) (layer B.Cu) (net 19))
 (segment (start 112.8347 102.6091) (end 117.7409 102.6091) (width 0.1524) (layer B.Cu) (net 19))
 (segment (start 111.959 101.7334) (end 112.8347 102.6091) (width 0.1524) (layer B.Cu) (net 19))
 (segment (start 111.959 99.4089) (end 111.959 101.7334) (width 0.1524) (layer B.Cu) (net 19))
 (segment (start 109.6342 97.0841) (end 111.959 99.4089) (width 0.1524) (layer B.Cu) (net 19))
 (segment (start 108.9075 97.0841) (end 109.6342 97.0841) (width 0.1524) (layer B.Cu) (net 19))
 (segment (start 108.476 96.6526) (end 108.9075 97.0841) (width 0.1524) (layer B.Cu) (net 19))
 (segment (start 108.275 94.5) (end 108.275 95.5289) (width 0.1524) (layer F.Cu) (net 19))
 (via (at 114.7398 100.5144) (size 0.6096) (layers F.Cu B.Cu) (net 10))
 (segment (start 114.7398 95.4502) (end 114.7398 100.5144) (width 0.1524) (layer B.Cu) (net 10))
 (segment (start 116.23 93.96) (end 114.7398 95.4502) (width 0.1524) (layer B.Cu) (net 10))
 (segment (start 108.2411 102.145) (end 107.625 101.5289) (width 0.1524) (layer F.Cu) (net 10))
 (segment (start 113.1092 102.145) (end 108.2411 102.145) (width 0.1524) (layer F.Cu) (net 10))
 (segment (start 114.7398 100.5144) (end 113.1092 102.145) (width 0.1524) (layer F.Cu) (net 10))
 (segment (start 107.625 100.5) (end 107.625 101.5289) (width 0.1524) (layer F.Cu) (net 10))
 (segment (start 109.575 100.5) (end 109.575 99.4711) (width 0.1524) (layer F.Cu) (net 11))
 (segment (start 117.6171 95.1129) (end 118.77 93.96) (width 0.1524) (layer F.Cu) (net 11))
 (segment (start 115.3519 95.1129) (end 117.6171 95.1129) (width 0.1524) (layer F.Cu) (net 11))
 (segment (start 110.9937 99.4711) (end 115.3519 95.1129) (width 0.1524) (layer F.Cu) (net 11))
 (segment (start 109.575 99.4711) (end 110.9937 99.4711) (width 0.1524) (layer F.Cu) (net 11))
 (segment (start 113.2589 99.4711) (end 112.175 99.4711) (width 0.1524) (layer F.Cu) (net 15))
 (segment (start 116.23 96.5) (end 113.2589 99.4711) (width 0.1524) (layer F.Cu) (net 15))
 (segment (start 112.175 100.5) (end 112.175 99.4711) (width 0.1524) (layer F.Cu) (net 15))
 (segment (start 115.5516 95.4445) (end 111.525 99.4711) (width 0.1524) (layer F.Cu) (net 14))
 (segment (start 117.7145 95.4445) (end 115.5516 95.4445) (width 0.1524) (layer F.Cu) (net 14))
 (segment (start 118.77 96.5) (end 117.7145 95.4445) (width 0.1524) (layer F.Cu) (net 14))
 (segment (start 111.525 100.5) (end 111.525 99.4711) (width 0.1524) (layer F.Cu) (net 14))
 (segment (start 110.875 100.5) (end 110.875 101.5289) (width 0.1524) (layer F.Cu) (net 13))
 (segment (start 112.539 101.5289) (end 110.875 101.5289) (width 0.1524) (layer F.Cu) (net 13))
 (segment (start 115.0279 99.04) (end 112.539 101.5289) (width 0.1524) (layer F.Cu) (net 13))
 (segment (start 116.23 99.04) (end 115.0279 99.04) (width 0.1524) (layer F.Cu) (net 13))
 (segment (start 110.225 100.5) (end 110.225 101.5289) (width 0.1524) (layer F.Cu) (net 12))
 (segment (start 110.5301 101.834) (end 110.225 101.5289) (width 0.1524) (layer F.Cu) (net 12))
 (segment (start 112.6655 101.834) (end 110.5301 101.834) (width 0.1524) (layer F.Cu) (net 12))
 (segment (start 114.5188 99.9807) (end 112.6655 101.834) (width 0.1524) (layer F.Cu) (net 12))
 (segment (start 114.961 99.9807) (end 114.5188 99.9807) (width 0.1524) (layer F.Cu) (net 12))
 (segment (start 115.089 100.1087) (end 114.961 99.9807) (width 0.1524) (layer F.Cu) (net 12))
 (segment (start 117.7013 100.1087) (end 115.089 100.1087) (width 0.1524) (layer F.Cu) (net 12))
 (segment (start 118.77 99.04) (end 117.7013 100.1087) (width 0.1524) (layer F.Cu) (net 12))
 (via (at 109.4758 97.7652) (size 0.6096) (layers F.Cu B.Cu) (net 8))
 (segment (start 110.225 94.5) (end 110.225 95.5289) (width 0.1524) (layer F.Cu) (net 8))
 (segment (start 98.639 97.266) (end 99.3251 97.266) (width 0.1524) (layer B.Cu) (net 8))
 (segment (start 99.8243 97.7652) (end 109.4758 97.7652) (width 0.1524) (layer B.Cu) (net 8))
 (segment (start 99.3251 97.266) (end 99.8243 97.7652) (width 0.1524) (layer B.Cu) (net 8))
 (segment (start 110.1812 97.0598) (end 109.4758 97.7652) (width 0.1524) (layer F.Cu) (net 8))
 (segment (start 110.1812 96.4927) (end 110.1812 97.0598) (width 0.1524) (layer F.Cu) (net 8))
 (segment (start 110.3621 96.3118) (end 110.1812 96.4927) (width 0.1524) (layer F.Cu) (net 8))
 (segment (start 110.3621 95.666) (end 110.3621 96.3118) (width 0.1524) (layer F.Cu) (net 8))
 (segment (start 110.225 95.5289) (end 110.3621 95.666) (width 0.1524) (layer F.Cu) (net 8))
 (via (at 106.711 99.2282) (size 0.6096) (layers F.Cu B.Cu) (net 9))
 (segment (start 105.6 99.2) (end 105.6 98.5711) (width 0.1524) (layer B.Cu) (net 9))
 (segment (start 111.405 101.5) (end 111.405 100.2711) (width 0.1524) (layer B.Cu) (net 9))
 (segment (start 106.9539 99.4711) (end 106.975 99.4711) (width 0.1524) (layer F.Cu) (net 9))
 (segment (start 106.711 99.2282) (end 106.9539 99.4711) (width 0.1524) (layer F.Cu) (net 9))
 (segment (start 106.975 100.5) (end 106.975 99.4711) (width 0.1524) (layer F.Cu) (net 9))
 (segment (start 105.6 98.5711) (end 106.711 98.5711) (width 0.1524) (layer B.Cu) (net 9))
 (segment (start 106.711 98.5711) (end 106.711 99.2282) (width 0.1524) (layer B.Cu) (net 9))
 (segment (start 111.405 99.2866) (end 111.405 100.2711) (width 0.1524) (layer B.Cu) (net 9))
 (segment (start 110.5122 98.3938) (end 111.405 99.2866) (width 0.1524) (layer B.Cu) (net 9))
 (segment (start 106.8883 98.3938) (end 110.5122 98.3938) (width 0.1524) (layer B.Cu) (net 9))
 (segment (start 106.711 98.5711) (end 106.8883 98.3938) (width 0.1524) (layer B.Cu) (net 9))
 (via (at 111.7286 93.0396) (size 0.6096) (layers F.Cu B.Cu) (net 16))
 (segment (start 111.4971 93.2711) (end 111.7286 93.0396) (width 0.1524) (layer B.Cu) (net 16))
 (segment (start 108.865 93.2711) (end 111.4971 93.2711) (width 0.1524) (layer B.Cu) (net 16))
 (segment (start 112.1601 93.4711) (end 112.175 93.4711) (width 0.1524) (layer F.Cu) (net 16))
 (segment (start 111.7286 93.0396) (end 112.1601 93.4711) (width 0.1524) (layer F.Cu) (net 16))
 (segment (start 112.175 94.5) (end 112.175 93.4711) (width 0.1524) (layer F.Cu) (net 16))
 (segment (start 108.865 94.5) (end 108.865 93.2711) (width 0.1524) (layer B.Cu) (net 16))
 (via (at 110.2839 98.9373) (size 0.6096) (layers F.Cu B.Cu) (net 17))
 (segment (start 110.135 101.5) (end 110.135 100.2711) (width 0.1524) (layer B.Cu) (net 17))
 (segment (start 110.2838 98.9373) (end 110.2839 98.9373) (width 0.1524) (layer B.Cu) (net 17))
 (segment (start 110.2838 100.1223) (end 110.2838 98.9373) (width 0.1524) (layer B.Cu) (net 17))
 (segment (start 110.135 100.2711) (end 110.2838 100.1223) (width 0.1524) (layer B.Cu) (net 17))
 (segment (start 111.525 94.5) (end 111.525 95.5289) (width 0.1524) (layer F.Cu) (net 17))
 (segment (start 111.525 97.6962) (end 111.525 95.5289) (width 0.1524) (layer F.Cu) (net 17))
 (segment (start 110.2839 98.9373) (end 111.525 97.6962) (width 0.1524) (layer F.Cu) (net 17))
 (via (at 110.7149 96.7138) (size 0.6096) (layers F.Cu B.Cu) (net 18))
 (segment (start 109.3888 96.7138) (end 110.7149 96.7138) (width 0.1524) (layer B.Cu) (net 18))
 (segment (start 108.4039 95.7289) (end 109.3888 96.7138) (width 0.1524) (layer B.Cu) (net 18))
 (segment (start 107.595 95.7289) (end 108.4039 95.7289) (width 0.1524) (layer B.Cu) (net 18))
 (segment (start 110.7149 95.689) (end 110.875 95.5289) (width 0.1524) (layer F.Cu) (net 18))
 (segment (start 110.7149 96.7138) (end 110.7149 95.689) (width 0.1524) (layer F.Cu) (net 18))
 (segment (start 110.875 94.5) (end 110.875 95.5289) (width 0.1524) (layer F.Cu) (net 18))
 (segment (start 107.595 94.5) (end 107.595 95.7289) (width 0.1524) (layer B.Cu) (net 18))
 (via (at 107.9141 99.085) (size 0.6096) (layers F.Cu B.Cu) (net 3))
 (segment (start 108.275 99.4459) (end 107.9141 99.085) (width 0.1524) (layer F.Cu) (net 3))
 (segment (start 108.275 100.5) (end 108.275 99.4459) (width 0.1524) (layer F.Cu) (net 3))
 (segment (start 105.878 101.1211) (end 105.5 101.1211) (width 0.1524) (layer B.Cu) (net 3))
 (segment (start 107.9141 99.085) (end 105.878 101.1211) (width 0.1524) (layer B.Cu) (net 3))
 (segment (start 105.5 101.75) (end 105.5 101.1211) (width 0.1524) (layer B.Cu) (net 3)))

